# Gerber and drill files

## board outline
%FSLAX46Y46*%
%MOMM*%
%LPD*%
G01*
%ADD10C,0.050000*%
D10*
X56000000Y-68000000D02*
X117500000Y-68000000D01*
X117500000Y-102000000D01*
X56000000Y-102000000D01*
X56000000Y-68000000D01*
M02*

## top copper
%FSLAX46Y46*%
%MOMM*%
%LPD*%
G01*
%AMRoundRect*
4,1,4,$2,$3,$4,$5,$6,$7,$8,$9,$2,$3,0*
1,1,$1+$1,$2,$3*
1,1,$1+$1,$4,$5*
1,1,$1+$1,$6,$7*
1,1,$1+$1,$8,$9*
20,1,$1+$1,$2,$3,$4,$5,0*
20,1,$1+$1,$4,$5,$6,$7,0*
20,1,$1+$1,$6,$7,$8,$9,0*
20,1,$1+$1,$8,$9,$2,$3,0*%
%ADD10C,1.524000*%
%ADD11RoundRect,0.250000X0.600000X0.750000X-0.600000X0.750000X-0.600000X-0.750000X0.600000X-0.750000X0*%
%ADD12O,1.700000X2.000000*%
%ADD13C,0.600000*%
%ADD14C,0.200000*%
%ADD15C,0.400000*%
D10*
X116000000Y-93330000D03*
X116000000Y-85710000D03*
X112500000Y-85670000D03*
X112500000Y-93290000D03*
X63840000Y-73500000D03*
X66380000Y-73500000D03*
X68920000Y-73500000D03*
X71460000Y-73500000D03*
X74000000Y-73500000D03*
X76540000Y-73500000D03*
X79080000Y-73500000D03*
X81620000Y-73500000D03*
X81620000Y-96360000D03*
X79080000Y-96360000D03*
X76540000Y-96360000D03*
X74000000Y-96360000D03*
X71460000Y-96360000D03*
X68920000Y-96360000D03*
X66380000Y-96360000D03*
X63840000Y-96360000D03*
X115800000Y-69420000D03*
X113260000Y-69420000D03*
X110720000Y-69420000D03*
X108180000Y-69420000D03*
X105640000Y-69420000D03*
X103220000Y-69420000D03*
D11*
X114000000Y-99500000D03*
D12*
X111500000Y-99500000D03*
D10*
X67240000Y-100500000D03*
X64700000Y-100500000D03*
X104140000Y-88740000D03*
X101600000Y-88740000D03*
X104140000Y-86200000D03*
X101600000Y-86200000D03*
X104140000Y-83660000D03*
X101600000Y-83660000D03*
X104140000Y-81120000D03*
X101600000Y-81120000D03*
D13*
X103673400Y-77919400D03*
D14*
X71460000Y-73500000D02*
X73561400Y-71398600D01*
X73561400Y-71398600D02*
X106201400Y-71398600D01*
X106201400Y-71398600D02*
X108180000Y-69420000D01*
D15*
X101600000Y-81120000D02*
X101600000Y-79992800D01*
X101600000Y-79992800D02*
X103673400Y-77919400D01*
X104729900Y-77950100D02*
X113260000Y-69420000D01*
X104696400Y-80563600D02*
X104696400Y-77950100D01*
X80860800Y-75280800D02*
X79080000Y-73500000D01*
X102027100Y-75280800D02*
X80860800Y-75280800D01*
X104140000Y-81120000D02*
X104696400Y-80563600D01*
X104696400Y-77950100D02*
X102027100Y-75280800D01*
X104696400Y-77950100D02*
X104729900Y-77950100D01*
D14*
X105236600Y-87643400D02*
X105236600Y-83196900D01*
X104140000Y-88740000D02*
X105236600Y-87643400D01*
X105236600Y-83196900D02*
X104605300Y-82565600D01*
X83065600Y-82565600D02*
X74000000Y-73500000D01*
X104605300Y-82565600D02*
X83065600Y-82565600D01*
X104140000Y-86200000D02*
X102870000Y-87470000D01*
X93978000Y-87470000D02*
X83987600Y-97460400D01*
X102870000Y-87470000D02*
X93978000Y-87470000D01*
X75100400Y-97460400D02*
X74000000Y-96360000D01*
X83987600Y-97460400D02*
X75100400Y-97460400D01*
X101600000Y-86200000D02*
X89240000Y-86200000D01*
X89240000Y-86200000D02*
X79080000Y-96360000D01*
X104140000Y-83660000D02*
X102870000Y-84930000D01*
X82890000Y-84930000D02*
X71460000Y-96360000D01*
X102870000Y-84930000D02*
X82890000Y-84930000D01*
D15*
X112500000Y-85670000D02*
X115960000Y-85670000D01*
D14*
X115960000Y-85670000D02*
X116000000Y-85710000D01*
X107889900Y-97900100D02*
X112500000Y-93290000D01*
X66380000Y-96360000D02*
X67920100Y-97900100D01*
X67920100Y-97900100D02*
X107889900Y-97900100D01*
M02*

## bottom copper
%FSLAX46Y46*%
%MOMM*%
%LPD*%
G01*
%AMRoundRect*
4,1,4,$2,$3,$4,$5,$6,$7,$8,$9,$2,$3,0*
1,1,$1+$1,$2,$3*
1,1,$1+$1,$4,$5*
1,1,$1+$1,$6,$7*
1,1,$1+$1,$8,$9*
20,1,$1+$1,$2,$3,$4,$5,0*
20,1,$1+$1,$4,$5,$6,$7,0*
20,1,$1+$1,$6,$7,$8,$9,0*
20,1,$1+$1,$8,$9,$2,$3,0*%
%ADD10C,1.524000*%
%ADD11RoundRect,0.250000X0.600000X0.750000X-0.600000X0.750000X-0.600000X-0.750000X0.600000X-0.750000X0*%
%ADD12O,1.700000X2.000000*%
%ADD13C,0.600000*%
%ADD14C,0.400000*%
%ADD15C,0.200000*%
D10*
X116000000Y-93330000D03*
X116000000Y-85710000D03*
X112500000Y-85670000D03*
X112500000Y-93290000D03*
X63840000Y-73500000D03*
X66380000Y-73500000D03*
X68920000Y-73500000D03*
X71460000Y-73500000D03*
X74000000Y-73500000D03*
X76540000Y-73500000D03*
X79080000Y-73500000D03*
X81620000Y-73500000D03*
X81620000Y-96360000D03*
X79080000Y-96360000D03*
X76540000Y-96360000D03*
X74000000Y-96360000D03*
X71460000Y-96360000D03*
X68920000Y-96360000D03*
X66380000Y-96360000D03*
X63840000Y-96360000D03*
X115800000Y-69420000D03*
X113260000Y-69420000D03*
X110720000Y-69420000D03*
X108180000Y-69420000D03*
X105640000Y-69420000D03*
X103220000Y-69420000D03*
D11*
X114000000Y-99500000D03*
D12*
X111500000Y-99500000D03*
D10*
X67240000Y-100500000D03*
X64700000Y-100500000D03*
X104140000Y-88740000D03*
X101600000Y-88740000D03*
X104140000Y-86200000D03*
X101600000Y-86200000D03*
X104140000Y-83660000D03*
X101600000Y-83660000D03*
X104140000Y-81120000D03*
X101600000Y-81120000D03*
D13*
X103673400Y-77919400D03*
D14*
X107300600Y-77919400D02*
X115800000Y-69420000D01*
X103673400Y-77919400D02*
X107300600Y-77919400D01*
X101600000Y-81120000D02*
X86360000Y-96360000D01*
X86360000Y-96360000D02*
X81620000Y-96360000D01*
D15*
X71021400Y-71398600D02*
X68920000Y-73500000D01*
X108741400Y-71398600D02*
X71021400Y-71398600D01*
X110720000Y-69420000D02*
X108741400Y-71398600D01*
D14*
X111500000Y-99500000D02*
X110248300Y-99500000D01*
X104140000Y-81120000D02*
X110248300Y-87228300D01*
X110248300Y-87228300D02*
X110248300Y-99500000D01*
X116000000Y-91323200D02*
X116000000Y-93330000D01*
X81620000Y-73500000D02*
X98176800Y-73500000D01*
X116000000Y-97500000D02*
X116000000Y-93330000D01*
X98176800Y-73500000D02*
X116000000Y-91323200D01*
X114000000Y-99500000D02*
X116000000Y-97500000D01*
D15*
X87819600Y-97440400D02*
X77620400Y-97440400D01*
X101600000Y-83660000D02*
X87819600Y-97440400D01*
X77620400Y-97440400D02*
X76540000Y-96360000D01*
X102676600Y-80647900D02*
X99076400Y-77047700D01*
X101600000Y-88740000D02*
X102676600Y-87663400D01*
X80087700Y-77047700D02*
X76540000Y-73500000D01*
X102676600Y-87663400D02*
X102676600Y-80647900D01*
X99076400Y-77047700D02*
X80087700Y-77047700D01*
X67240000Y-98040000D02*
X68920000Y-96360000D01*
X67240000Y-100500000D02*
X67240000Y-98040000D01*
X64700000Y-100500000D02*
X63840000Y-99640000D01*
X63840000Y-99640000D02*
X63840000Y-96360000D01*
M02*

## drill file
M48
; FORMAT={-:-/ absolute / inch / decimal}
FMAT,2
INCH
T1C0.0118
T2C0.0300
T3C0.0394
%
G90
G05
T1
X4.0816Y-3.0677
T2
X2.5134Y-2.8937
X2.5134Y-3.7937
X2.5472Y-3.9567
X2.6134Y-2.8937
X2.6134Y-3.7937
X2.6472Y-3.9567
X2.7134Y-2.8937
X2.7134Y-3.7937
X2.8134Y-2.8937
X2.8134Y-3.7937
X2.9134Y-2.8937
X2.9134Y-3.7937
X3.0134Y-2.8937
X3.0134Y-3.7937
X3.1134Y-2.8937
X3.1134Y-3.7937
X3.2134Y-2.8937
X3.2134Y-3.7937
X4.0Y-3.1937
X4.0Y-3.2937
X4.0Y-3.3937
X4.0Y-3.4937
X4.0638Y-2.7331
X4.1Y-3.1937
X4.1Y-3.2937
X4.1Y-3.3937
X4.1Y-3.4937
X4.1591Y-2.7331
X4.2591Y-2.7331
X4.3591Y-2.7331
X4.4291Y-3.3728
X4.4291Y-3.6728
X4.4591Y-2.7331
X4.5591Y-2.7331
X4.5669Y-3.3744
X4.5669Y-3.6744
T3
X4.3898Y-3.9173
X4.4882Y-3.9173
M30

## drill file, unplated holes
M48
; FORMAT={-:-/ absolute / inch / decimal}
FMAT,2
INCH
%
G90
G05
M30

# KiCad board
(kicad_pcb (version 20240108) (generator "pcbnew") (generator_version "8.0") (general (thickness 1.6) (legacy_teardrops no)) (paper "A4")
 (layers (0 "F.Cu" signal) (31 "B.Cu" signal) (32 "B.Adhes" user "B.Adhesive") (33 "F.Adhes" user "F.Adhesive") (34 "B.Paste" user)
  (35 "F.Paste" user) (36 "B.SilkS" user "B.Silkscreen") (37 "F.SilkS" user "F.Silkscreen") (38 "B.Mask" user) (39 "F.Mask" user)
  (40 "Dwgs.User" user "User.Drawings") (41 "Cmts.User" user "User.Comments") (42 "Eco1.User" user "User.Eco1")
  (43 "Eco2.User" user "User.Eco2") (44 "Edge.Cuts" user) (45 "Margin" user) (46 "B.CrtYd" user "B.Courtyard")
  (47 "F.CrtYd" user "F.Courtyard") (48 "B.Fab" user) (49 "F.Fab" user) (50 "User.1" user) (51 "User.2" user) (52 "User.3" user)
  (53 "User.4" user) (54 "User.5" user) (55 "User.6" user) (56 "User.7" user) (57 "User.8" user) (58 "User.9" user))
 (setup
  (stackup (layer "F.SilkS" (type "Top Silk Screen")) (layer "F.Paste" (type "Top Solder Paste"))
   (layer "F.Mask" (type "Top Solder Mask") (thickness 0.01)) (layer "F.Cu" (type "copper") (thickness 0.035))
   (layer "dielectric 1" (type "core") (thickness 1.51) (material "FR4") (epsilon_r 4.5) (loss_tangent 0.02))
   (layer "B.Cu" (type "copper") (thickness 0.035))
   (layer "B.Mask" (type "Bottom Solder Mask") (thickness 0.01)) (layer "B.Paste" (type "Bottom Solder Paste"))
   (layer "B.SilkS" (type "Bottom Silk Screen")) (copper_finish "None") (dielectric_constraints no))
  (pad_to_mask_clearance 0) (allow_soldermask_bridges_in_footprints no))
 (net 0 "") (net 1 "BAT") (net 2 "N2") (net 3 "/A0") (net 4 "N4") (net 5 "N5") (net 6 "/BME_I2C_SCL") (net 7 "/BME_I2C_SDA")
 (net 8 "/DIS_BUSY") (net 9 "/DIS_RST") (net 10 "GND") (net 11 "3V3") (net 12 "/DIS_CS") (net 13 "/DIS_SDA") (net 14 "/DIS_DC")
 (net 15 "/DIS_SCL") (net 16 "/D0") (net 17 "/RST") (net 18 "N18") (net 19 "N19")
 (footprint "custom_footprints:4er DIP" (layer "F.Cu") (at 116 88.25 180)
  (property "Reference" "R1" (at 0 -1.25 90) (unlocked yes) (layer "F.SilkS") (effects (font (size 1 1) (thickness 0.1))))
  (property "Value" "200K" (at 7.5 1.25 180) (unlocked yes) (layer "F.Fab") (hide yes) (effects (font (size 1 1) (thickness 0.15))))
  (pad "1" thru_hole circle (at 0 -5.08 180) (size 1.524 1.524) (drill 0.762) (layers "*.Cu" "*.Mask") (remove_unused_layers no)
   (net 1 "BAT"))
  (pad "2" thru_hole circle (at 0 2.54 180) (size 1.524 1.524) (drill 0.762) (layers "*.Cu" "*.Mask") (remove_unused_layers no) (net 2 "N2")))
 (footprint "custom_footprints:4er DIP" (layer "F.Cu") (at 112.5 90.75)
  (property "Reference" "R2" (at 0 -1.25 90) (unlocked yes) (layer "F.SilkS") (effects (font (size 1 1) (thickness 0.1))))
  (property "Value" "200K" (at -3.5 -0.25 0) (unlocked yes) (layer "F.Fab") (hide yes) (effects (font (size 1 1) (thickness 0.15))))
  (pad "1" thru_hole circle (at 0 -5.08) (size 1.524 1.524) (drill 0.762) (layers "*.Cu" "*.Mask") (remove_unused_layers no) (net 2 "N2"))
  (pad "2" thru_hole circle (at 0 2.54) (size 1.524 1.524) (drill 0.762) (layers "*.Cu" "*.Mask") (remove_unused_layers no) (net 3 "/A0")))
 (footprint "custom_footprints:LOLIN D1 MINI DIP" (layer "F.Cu") (at 74 83.66 90)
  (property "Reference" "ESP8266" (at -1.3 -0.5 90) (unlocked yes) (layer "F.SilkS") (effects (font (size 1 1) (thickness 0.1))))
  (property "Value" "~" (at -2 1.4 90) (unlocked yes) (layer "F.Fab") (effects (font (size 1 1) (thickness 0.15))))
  (pad "1" thru_hole circle (at 10.16 -10.16 90) (size 1.524 1.524) (drill 0.762) (layers "*.Cu" "*.Mask") (remove_unused_layers no)
   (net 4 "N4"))
  (pad "2" thru_hole circle (at 10.16 -7.62 90) (size 1.524 1.524) (drill 0.762) (layers "*.Cu" "*.Mask") (remove_unused_layers no)
   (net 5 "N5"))
  (pad "3" thru_hole circle (at 10.16 -5.08 90) (size 1.524 1.524) (drill 0.762) (layers "*.Cu" "*.Mask") (remove_unused_layers no)
   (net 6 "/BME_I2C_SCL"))
  (pad "4" thru_hole circle (at 10.16 -2.54 90) (size 1.524 1.524) (drill 0.762) (layers "*.Cu" "*.Mask") (remove_unused_layers no)
   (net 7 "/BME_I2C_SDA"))
  (pad "5" thru_hole circle (at 10.16 0 90) (size 1.524 1.524) (drill 0.762) (layers "*.Cu" "*.Mask") (remove_unused_layers no)
   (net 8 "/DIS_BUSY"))
  (pad "6" thru_hole circle (at 10.16 2.54 90) (size 1.524 1.524) (drill 0.762) (layers "*.Cu" "*.Mask") (remove_unused_layers no)
   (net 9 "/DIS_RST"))
  (pad "7" thru_hole circle (at 10.16 5.08 90) (size 1.524 1.524) (drill 0.762) (layers "*.Cu" "*.Mask") (remove_unused_layers no)
   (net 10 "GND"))
  (pad "8" thru_hole circle (at 10.16 7.62 90) (size 1.524 1.524) (drill 0.762) (layers "*.Cu" "*.Mask") (remove_unused_layers no)
   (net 1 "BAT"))
  (pad "9" thru_hole circle (at -12.7 7.62 90) (size 1.524 1.524) (drill 0.762) (layers "*.Cu" "*.Mask") (remove_unused_layers no)
   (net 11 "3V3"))
  (pad "10" thru_hole circle (at -12.7 5.08 90) (size 1.524 1.524) (drill 0.762) (layers "*.Cu" "*.Mask") (remove_unused_layers no)
   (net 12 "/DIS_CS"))
  (pad "11" thru_hole circle (at -12.7 2.54 90) (size 1.524 1.524) (drill 0.762) (layers "*.Cu" "*.Mask") (remove_unused_layers no)
   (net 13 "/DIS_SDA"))
  (pad "12" thru_hole circle (at -12.7 0 90) (size 1.524 1.524) (drill 0.762) (layers "*.Cu" "*.Mask") (remove_unused_layers no)
   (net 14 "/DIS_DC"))
  (pad "13" thru_hole circle (at -12.7 -2.54 90) (size 1.524 1.524) (drill 0.762) (layers "*.Cu" "*.Mask") (remove_unused_layers no)
   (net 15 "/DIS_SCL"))
  (pad "14" thru_hole circle (at -12.7 -5.08 90) (size 1.524 1.524) (drill 0.762) (layers "*.Cu" "*.Mask") (remove_unused_layers no)
   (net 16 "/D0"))
  (pad "15" thru_hole circle (at -12.7 -7.62 90) (size 1.524 1.524) (drill 0.762) (layers "*.Cu" "*.Mask") (remove_unused_layers no)
   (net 3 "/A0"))
  (pad "16" thru_hole circle (at -12.7 -10.16 90) (size 1.524 1.524) (drill 0.762) (layers "*.Cu" "*.Mask") (remove_unused_layers no)
   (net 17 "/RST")))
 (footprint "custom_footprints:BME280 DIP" (layer "F.Cu") (at 108.3 74.5)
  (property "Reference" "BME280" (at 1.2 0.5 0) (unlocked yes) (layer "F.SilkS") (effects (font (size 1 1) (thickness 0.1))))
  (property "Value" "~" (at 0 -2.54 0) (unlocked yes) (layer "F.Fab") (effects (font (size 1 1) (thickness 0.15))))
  (pad "1" thru_hole circle (at 7.5 -5.08) (size 1.524 1.524) (drill 0.762) (layers "*.Cu" "*.Mask") (remove_unused_layers no)
   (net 11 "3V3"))
  (pad "2" thru_hole circle (at 4.96 -5.08) (size 1.524 1.524) (drill 0.762) (layers "*.Cu" "*.Mask") (remove_unused_layers no)
   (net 10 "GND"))
  (pad "3" thru_hole circle (at 2.42 -5.08) (size 1.524 1.524) (drill 0.762) (layers "*.Cu" "*.Mask") (remove_unused_layers no)
   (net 6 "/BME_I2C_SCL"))
  (pad "4" thru_hole circle (at -0.12 -5.08) (size 1.524 1.524) (drill 0.762) (layers "*.Cu" "*.Mask") (remove_unused_layers no)
   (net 7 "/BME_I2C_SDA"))
  (pad "5" thru_hole circle (at -2.66 -5.08) (size 1.524 1.524) (drill 0.762) (layers "*.Cu" "*.Mask") (remove_unused_layers no)
   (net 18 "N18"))
  (pad "6" thru_hole circle (at -5.08 -5.08) (size 1.524 1.524) (drill 0.762) (layers "*.Cu" "*.Mask") (remove_unused_layers no)
   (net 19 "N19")))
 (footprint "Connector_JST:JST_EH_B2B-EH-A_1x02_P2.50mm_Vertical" (layer "F.Cu") (at 114 99.5 180)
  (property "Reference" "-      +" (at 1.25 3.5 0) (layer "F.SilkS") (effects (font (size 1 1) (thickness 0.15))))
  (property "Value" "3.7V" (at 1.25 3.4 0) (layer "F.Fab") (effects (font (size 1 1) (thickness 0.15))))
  (pad "1" thru_hole roundrect (at 0 0 180) (size 1.7 2) (drill 1) (layers "*.Cu" "*.Mask") (remove_unused_layers no)
   (roundrect_rratio 0.147059) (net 1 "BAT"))
  (pad "2" thru_hole oval (at 2.5 0 180) (size 1.7 2) (drill 1) (layers "*.Cu" "*.Mask") (remove_unused_layers no) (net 10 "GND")))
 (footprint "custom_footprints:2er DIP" (layer "F.Cu") (at 64.7 100.5 -90)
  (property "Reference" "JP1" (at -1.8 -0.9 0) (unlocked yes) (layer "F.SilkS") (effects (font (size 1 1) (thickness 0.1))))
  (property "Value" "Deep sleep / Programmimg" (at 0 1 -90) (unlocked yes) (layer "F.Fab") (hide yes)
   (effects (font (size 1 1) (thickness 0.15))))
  (pad "1" thru_hole circle (at 0 -2.54 270) (size 1.524 1.524) (drill 0.762) (layers "*.Cu" "*.Mask") (remove_unused_layers no)
   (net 16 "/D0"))
  (pad "2" thru_hole circle (at 0 0 270) (size 1.524 1.524) (drill 0.762) (layers "*.Cu" "*.Mask") (remove_unused_layers no) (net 17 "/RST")))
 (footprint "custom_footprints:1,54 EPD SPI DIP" (layer "B.Cu") (at 81.5 85)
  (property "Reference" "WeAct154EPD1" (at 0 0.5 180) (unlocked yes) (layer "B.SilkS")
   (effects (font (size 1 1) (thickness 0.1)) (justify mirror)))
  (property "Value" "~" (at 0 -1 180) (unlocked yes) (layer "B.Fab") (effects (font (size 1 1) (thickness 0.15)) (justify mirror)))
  (pad "1" thru_hole circle (at 22.64 3.74) (size 1.524 1.524) (drill 0.762) (layers "*.Cu" "*.Mask") (remove_unused_layers no)
   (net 8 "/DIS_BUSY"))
  (pad "2" thru_hole circle (at 20.1 3.74) (size 1.524 1.524) (drill 0.762) (layers "*.Cu" "*.Mask") (remove_unused_layers no)
   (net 9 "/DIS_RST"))
  (pad "3" thru_hole circle (at 22.64 1.2) (size 1.524 1.524) (drill 0.762) (layers "*.Cu" "*.Mask") (remove_unused_layers no)
   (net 14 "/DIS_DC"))
  (pad "4" thru_hole circle (at 20.1 1.2) (size 1.524 1.524) (drill 0.762) (layers "*.Cu" "*.Mask") (remove_unused_layers no)
   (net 12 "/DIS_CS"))
  (pad "5" thru_hole circle (at 22.64 -1.34) (size 1.524 1.524) (drill 0.762) (layers "*.Cu" "*.Mask") (remove_unused_layers no)
   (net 15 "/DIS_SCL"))
  (pad "6" thru_hole circle (at 20.1 -1.34) (size 1.524 1.524) (drill 0.762) (layers "*.Cu" "*.Mask") (remove_unused_layers no)
   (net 13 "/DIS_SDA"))
  (pad "7" thru_hole circle (at 22.64 -3.88) (size 1.524 1.524) (drill 0.762) (layers "*.Cu" "*.Mask") (remove_unused_layers no)
   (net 10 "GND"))
  (pad "8" thru_hole circle (at 20.1 -3.88) (size 1.524 1.524) (drill 0.762) (layers "*.Cu" "*.Mask") (remove_unused_layers no)
   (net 11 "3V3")))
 (gr_rect (start 56 68) (end 117.5 102) (stroke (width 0.05) (type default)) (fill none) (layer "Edge.Cuts"))
 (segment (start 71.46 73.5) (end 73.5614 71.3986) (width 0.2) (layer "F.Cu") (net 7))
 (segment (start 73.5614 71.3986) (end 106.2014 71.3986) (width 0.2) (layer "F.Cu") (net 7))
 (segment (start 106.2014 71.3986) (end 108.18 69.42) (width 0.2) (layer "F.Cu") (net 7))
 (segment (start 101.6 81.12) (end 101.6 79.9928) (width 0.4) (layer "F.Cu") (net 11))
 (segment (start 101.6 79.9928) (end 103.6734 77.9194) (width 0.4) (layer "F.Cu") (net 11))
 (via (at 103.6734 77.9194) (size 0.6) (drill 0.3) (layers "F.Cu" "B.Cu") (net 11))
 (segment (start 107.3006 77.9194) (end 115.8 69.42) (width 0.4) (layer "B.Cu") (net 11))
 (segment (start 103.6734 77.9194) (end 107.3006 77.9194) (width 0.4) (layer "B.Cu") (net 11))
 (segment (start 101.6 81.12) (end 86.36 96.36) (width 0.4) (layer "B.Cu") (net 11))
 (segment (start 86.36 96.36) (end 81.62 96.36) (width 0.4) (layer "B.Cu") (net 11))
 (segment (start 71.0214 71.3986) (end 68.92 73.5) (width 0.2) (layer "B.Cu") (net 6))
 (segment (start 108.7414 71.3986) (end 71.0214 71.3986) (width 0.2) (layer "B.Cu") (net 6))
 (segment (start 110.72 69.42) (end 108.7414 71.3986) (width 0.2) (layer "B.Cu") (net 6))
 (segment (start 104.7299 77.9501) (end 113.26 69.42) (width 0.4) (layer "F.Cu") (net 10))
 (segment (start 104.6964 80.5636) (end 104.6964 77.9501) (width 0.4) (layer "F.Cu") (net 10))
 (segment (start 80.8608 75.2808) (end 79.08 73.5) (width 0.4) (layer "F.Cu") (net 10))
 (segment (start 102.0271 75.2808) (end 80.8608 75.2808) (width 0.4) (layer "F.Cu") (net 10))
 (segment (start 104.14 81.12) (end 104.6964 80.5636) (width 0.4) (layer "F.Cu") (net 10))
 (segment (start 104.6964 77.9501) (end 102.0271 75.2808) (width 0.4) (layer "F.Cu") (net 10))
 (segment (start 104.6964 77.9501) (end 104.7299 77.9501) (width 0.4) (layer "F.Cu") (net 10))
 (segment (start 111.5 99.5) (end 110.2483 99.5) (width 0.4) (layer "B.Cu") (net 10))
 (segment (start 104.14 81.12) (end 110.2483 87.2283) (width 0.4) (layer "B.Cu") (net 10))
 (segment (start 110.2483 87.2283) (end 110.2483 99.5) (width 0.4) (layer "B.Cu") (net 10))
 (segment (start 116 91.3232) (end 116 93.33) (width 0.4) (layer "B.Cu") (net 1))
 (segment (start 81.62 73.5) (end 98.1768 73.5) (width 0.4) (layer "B.Cu") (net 1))
 (segment (start 116 97.5) (end 116 93.33) (width 0.4) (layer "B.Cu") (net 1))
 (segment (start 98.1768 73.5) (end 116 91.3232) (width 0.4) (layer "B.Cu") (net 1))
 (segment (start 114 99.5) (end 116 97.5) (width 0.4) (layer "B.Cu") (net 1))
 (segment (start 87.8196 97.4404) (end 77.6204 97.4404) (width 0.2) (layer "B.Cu") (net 13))
 (segment (start 101.6 83.66) (end 87.8196 97.4404) (width 0.2) (layer "B.Cu") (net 13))
 (segment (start 77.6204 97.4404) (end 76.54 96.36) (width 0.2) (layer "B.Cu") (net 13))
 (segment (start 105.2366 87.6434) (end 105.2366 83.1969) (width 0.2) (layer "F.Cu") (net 8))
 (segment (start 104.14 88.74) (end 105.2366 87.6434) (width 0.2) (layer "F.Cu") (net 8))
 (segment (start 105.2366 83.1969) (end 104.6053 82.5656) (width 0.2) (layer "F.Cu") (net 8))
 (segment (start 83.0656 82.5656) (end 74 73.5) (width 0.2) (layer "F.Cu") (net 8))
 (segment (start 104.6053 82.5656) (end 83.0656 82.5656) (width 0.2) (layer "F.Cu") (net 8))
 (segment (start 102.6766 80.6479) (end 99.0764 77.0477) (width 0.2) (layer "B.Cu") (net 9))
 (segment (start 101.6 88.74) (end 102.6766 87.6634) (width 0.2) (layer "B.Cu") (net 9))
 (segment (start 80.0877 77.0477) (end 76.54 73.5) (width 0.2) (layer "B.Cu") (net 9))
 (segment (start 102.6766 87.6634) (end 102.6766 80.6479) (width 0.2) (layer "B.Cu") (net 9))
 (segment (start 99.0764 77.0477) (end 80.0877 77.0477) (width 0.2) (layer "B.Cu") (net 9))
 (segment (start 104.14 86.2) (end 102.87 87.47) (width 0.2) (layer "F.Cu") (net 14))
 (segment (start 93.978 87.47) (end 83.9876 97.4604) (width 0.2) (layer "F.Cu") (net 14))
 (segment (start 102.87 87.47) (end 93.978 87.47) (width 0.2) (layer "F.Cu") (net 14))
 (segment (start 75.1004 97.4604) (end 74 96.36) (width 0.2) (layer "F.Cu") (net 14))
 (segment (start 83.9876 97.4604) (end 75.1004 97.4604) (width 0.2) (layer "F.Cu") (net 14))
 (segment (start 101.6 86.2) (end 89.24 86.2) (width 0.2) (layer "F.Cu") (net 12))
 (segment (start 89.24 86.2) (end 79.08 96.36) (width 0.2) (layer "F.Cu") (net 12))
 (segment (start 104.14 83.66) (end 102.87 84.93) (width 0.2) (layer "F.Cu") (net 15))
 (segment (start 82.89 84.93) (end 71.46 96.36) (width 0.2) (layer "F.Cu") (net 15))
 (segment (start 102.87 84.93) (end 82.89 84.93) (width 0.2) (layer "F.Cu") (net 15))
 (segment (start 67.24 98.04) (end 68.92 96.36) (width 0.2) (layer "B.Cu") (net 16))
 (segment (start 67.24 100.5) (end 67.24 98.04) (width 0.2) (layer "B.Cu") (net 16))
 (segment (start 64.7 100.5) (end 63.84 99.64) (width 0.2) (layer "B.Cu") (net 17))
 (segment (start 63.84 99.64) (end 63.84 96.36) (width 0.2) (layer "B.Cu") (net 17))
 (segment (start 112.5 85.67) (end 115.96 85.67) (width 0.4) (layer "F.Cu") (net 2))
 (segment (start 115.96 85.67) (end 116 85.71) (width 0.2) (layer "F.Cu") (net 2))
 (segment (start 107.8899 97.9001) (end 112.5 93.29) (width 0.2) (layer "F.Cu") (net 3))
 (segment (start 66.38 96.36) (end 67.9201 97.9001) (width 0.2) (layer "F.Cu") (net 3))
 (segment (start 67.9201 97.9001) (end 107.8899 97.9001) (width 0.2) (layer "F.Cu") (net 3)))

